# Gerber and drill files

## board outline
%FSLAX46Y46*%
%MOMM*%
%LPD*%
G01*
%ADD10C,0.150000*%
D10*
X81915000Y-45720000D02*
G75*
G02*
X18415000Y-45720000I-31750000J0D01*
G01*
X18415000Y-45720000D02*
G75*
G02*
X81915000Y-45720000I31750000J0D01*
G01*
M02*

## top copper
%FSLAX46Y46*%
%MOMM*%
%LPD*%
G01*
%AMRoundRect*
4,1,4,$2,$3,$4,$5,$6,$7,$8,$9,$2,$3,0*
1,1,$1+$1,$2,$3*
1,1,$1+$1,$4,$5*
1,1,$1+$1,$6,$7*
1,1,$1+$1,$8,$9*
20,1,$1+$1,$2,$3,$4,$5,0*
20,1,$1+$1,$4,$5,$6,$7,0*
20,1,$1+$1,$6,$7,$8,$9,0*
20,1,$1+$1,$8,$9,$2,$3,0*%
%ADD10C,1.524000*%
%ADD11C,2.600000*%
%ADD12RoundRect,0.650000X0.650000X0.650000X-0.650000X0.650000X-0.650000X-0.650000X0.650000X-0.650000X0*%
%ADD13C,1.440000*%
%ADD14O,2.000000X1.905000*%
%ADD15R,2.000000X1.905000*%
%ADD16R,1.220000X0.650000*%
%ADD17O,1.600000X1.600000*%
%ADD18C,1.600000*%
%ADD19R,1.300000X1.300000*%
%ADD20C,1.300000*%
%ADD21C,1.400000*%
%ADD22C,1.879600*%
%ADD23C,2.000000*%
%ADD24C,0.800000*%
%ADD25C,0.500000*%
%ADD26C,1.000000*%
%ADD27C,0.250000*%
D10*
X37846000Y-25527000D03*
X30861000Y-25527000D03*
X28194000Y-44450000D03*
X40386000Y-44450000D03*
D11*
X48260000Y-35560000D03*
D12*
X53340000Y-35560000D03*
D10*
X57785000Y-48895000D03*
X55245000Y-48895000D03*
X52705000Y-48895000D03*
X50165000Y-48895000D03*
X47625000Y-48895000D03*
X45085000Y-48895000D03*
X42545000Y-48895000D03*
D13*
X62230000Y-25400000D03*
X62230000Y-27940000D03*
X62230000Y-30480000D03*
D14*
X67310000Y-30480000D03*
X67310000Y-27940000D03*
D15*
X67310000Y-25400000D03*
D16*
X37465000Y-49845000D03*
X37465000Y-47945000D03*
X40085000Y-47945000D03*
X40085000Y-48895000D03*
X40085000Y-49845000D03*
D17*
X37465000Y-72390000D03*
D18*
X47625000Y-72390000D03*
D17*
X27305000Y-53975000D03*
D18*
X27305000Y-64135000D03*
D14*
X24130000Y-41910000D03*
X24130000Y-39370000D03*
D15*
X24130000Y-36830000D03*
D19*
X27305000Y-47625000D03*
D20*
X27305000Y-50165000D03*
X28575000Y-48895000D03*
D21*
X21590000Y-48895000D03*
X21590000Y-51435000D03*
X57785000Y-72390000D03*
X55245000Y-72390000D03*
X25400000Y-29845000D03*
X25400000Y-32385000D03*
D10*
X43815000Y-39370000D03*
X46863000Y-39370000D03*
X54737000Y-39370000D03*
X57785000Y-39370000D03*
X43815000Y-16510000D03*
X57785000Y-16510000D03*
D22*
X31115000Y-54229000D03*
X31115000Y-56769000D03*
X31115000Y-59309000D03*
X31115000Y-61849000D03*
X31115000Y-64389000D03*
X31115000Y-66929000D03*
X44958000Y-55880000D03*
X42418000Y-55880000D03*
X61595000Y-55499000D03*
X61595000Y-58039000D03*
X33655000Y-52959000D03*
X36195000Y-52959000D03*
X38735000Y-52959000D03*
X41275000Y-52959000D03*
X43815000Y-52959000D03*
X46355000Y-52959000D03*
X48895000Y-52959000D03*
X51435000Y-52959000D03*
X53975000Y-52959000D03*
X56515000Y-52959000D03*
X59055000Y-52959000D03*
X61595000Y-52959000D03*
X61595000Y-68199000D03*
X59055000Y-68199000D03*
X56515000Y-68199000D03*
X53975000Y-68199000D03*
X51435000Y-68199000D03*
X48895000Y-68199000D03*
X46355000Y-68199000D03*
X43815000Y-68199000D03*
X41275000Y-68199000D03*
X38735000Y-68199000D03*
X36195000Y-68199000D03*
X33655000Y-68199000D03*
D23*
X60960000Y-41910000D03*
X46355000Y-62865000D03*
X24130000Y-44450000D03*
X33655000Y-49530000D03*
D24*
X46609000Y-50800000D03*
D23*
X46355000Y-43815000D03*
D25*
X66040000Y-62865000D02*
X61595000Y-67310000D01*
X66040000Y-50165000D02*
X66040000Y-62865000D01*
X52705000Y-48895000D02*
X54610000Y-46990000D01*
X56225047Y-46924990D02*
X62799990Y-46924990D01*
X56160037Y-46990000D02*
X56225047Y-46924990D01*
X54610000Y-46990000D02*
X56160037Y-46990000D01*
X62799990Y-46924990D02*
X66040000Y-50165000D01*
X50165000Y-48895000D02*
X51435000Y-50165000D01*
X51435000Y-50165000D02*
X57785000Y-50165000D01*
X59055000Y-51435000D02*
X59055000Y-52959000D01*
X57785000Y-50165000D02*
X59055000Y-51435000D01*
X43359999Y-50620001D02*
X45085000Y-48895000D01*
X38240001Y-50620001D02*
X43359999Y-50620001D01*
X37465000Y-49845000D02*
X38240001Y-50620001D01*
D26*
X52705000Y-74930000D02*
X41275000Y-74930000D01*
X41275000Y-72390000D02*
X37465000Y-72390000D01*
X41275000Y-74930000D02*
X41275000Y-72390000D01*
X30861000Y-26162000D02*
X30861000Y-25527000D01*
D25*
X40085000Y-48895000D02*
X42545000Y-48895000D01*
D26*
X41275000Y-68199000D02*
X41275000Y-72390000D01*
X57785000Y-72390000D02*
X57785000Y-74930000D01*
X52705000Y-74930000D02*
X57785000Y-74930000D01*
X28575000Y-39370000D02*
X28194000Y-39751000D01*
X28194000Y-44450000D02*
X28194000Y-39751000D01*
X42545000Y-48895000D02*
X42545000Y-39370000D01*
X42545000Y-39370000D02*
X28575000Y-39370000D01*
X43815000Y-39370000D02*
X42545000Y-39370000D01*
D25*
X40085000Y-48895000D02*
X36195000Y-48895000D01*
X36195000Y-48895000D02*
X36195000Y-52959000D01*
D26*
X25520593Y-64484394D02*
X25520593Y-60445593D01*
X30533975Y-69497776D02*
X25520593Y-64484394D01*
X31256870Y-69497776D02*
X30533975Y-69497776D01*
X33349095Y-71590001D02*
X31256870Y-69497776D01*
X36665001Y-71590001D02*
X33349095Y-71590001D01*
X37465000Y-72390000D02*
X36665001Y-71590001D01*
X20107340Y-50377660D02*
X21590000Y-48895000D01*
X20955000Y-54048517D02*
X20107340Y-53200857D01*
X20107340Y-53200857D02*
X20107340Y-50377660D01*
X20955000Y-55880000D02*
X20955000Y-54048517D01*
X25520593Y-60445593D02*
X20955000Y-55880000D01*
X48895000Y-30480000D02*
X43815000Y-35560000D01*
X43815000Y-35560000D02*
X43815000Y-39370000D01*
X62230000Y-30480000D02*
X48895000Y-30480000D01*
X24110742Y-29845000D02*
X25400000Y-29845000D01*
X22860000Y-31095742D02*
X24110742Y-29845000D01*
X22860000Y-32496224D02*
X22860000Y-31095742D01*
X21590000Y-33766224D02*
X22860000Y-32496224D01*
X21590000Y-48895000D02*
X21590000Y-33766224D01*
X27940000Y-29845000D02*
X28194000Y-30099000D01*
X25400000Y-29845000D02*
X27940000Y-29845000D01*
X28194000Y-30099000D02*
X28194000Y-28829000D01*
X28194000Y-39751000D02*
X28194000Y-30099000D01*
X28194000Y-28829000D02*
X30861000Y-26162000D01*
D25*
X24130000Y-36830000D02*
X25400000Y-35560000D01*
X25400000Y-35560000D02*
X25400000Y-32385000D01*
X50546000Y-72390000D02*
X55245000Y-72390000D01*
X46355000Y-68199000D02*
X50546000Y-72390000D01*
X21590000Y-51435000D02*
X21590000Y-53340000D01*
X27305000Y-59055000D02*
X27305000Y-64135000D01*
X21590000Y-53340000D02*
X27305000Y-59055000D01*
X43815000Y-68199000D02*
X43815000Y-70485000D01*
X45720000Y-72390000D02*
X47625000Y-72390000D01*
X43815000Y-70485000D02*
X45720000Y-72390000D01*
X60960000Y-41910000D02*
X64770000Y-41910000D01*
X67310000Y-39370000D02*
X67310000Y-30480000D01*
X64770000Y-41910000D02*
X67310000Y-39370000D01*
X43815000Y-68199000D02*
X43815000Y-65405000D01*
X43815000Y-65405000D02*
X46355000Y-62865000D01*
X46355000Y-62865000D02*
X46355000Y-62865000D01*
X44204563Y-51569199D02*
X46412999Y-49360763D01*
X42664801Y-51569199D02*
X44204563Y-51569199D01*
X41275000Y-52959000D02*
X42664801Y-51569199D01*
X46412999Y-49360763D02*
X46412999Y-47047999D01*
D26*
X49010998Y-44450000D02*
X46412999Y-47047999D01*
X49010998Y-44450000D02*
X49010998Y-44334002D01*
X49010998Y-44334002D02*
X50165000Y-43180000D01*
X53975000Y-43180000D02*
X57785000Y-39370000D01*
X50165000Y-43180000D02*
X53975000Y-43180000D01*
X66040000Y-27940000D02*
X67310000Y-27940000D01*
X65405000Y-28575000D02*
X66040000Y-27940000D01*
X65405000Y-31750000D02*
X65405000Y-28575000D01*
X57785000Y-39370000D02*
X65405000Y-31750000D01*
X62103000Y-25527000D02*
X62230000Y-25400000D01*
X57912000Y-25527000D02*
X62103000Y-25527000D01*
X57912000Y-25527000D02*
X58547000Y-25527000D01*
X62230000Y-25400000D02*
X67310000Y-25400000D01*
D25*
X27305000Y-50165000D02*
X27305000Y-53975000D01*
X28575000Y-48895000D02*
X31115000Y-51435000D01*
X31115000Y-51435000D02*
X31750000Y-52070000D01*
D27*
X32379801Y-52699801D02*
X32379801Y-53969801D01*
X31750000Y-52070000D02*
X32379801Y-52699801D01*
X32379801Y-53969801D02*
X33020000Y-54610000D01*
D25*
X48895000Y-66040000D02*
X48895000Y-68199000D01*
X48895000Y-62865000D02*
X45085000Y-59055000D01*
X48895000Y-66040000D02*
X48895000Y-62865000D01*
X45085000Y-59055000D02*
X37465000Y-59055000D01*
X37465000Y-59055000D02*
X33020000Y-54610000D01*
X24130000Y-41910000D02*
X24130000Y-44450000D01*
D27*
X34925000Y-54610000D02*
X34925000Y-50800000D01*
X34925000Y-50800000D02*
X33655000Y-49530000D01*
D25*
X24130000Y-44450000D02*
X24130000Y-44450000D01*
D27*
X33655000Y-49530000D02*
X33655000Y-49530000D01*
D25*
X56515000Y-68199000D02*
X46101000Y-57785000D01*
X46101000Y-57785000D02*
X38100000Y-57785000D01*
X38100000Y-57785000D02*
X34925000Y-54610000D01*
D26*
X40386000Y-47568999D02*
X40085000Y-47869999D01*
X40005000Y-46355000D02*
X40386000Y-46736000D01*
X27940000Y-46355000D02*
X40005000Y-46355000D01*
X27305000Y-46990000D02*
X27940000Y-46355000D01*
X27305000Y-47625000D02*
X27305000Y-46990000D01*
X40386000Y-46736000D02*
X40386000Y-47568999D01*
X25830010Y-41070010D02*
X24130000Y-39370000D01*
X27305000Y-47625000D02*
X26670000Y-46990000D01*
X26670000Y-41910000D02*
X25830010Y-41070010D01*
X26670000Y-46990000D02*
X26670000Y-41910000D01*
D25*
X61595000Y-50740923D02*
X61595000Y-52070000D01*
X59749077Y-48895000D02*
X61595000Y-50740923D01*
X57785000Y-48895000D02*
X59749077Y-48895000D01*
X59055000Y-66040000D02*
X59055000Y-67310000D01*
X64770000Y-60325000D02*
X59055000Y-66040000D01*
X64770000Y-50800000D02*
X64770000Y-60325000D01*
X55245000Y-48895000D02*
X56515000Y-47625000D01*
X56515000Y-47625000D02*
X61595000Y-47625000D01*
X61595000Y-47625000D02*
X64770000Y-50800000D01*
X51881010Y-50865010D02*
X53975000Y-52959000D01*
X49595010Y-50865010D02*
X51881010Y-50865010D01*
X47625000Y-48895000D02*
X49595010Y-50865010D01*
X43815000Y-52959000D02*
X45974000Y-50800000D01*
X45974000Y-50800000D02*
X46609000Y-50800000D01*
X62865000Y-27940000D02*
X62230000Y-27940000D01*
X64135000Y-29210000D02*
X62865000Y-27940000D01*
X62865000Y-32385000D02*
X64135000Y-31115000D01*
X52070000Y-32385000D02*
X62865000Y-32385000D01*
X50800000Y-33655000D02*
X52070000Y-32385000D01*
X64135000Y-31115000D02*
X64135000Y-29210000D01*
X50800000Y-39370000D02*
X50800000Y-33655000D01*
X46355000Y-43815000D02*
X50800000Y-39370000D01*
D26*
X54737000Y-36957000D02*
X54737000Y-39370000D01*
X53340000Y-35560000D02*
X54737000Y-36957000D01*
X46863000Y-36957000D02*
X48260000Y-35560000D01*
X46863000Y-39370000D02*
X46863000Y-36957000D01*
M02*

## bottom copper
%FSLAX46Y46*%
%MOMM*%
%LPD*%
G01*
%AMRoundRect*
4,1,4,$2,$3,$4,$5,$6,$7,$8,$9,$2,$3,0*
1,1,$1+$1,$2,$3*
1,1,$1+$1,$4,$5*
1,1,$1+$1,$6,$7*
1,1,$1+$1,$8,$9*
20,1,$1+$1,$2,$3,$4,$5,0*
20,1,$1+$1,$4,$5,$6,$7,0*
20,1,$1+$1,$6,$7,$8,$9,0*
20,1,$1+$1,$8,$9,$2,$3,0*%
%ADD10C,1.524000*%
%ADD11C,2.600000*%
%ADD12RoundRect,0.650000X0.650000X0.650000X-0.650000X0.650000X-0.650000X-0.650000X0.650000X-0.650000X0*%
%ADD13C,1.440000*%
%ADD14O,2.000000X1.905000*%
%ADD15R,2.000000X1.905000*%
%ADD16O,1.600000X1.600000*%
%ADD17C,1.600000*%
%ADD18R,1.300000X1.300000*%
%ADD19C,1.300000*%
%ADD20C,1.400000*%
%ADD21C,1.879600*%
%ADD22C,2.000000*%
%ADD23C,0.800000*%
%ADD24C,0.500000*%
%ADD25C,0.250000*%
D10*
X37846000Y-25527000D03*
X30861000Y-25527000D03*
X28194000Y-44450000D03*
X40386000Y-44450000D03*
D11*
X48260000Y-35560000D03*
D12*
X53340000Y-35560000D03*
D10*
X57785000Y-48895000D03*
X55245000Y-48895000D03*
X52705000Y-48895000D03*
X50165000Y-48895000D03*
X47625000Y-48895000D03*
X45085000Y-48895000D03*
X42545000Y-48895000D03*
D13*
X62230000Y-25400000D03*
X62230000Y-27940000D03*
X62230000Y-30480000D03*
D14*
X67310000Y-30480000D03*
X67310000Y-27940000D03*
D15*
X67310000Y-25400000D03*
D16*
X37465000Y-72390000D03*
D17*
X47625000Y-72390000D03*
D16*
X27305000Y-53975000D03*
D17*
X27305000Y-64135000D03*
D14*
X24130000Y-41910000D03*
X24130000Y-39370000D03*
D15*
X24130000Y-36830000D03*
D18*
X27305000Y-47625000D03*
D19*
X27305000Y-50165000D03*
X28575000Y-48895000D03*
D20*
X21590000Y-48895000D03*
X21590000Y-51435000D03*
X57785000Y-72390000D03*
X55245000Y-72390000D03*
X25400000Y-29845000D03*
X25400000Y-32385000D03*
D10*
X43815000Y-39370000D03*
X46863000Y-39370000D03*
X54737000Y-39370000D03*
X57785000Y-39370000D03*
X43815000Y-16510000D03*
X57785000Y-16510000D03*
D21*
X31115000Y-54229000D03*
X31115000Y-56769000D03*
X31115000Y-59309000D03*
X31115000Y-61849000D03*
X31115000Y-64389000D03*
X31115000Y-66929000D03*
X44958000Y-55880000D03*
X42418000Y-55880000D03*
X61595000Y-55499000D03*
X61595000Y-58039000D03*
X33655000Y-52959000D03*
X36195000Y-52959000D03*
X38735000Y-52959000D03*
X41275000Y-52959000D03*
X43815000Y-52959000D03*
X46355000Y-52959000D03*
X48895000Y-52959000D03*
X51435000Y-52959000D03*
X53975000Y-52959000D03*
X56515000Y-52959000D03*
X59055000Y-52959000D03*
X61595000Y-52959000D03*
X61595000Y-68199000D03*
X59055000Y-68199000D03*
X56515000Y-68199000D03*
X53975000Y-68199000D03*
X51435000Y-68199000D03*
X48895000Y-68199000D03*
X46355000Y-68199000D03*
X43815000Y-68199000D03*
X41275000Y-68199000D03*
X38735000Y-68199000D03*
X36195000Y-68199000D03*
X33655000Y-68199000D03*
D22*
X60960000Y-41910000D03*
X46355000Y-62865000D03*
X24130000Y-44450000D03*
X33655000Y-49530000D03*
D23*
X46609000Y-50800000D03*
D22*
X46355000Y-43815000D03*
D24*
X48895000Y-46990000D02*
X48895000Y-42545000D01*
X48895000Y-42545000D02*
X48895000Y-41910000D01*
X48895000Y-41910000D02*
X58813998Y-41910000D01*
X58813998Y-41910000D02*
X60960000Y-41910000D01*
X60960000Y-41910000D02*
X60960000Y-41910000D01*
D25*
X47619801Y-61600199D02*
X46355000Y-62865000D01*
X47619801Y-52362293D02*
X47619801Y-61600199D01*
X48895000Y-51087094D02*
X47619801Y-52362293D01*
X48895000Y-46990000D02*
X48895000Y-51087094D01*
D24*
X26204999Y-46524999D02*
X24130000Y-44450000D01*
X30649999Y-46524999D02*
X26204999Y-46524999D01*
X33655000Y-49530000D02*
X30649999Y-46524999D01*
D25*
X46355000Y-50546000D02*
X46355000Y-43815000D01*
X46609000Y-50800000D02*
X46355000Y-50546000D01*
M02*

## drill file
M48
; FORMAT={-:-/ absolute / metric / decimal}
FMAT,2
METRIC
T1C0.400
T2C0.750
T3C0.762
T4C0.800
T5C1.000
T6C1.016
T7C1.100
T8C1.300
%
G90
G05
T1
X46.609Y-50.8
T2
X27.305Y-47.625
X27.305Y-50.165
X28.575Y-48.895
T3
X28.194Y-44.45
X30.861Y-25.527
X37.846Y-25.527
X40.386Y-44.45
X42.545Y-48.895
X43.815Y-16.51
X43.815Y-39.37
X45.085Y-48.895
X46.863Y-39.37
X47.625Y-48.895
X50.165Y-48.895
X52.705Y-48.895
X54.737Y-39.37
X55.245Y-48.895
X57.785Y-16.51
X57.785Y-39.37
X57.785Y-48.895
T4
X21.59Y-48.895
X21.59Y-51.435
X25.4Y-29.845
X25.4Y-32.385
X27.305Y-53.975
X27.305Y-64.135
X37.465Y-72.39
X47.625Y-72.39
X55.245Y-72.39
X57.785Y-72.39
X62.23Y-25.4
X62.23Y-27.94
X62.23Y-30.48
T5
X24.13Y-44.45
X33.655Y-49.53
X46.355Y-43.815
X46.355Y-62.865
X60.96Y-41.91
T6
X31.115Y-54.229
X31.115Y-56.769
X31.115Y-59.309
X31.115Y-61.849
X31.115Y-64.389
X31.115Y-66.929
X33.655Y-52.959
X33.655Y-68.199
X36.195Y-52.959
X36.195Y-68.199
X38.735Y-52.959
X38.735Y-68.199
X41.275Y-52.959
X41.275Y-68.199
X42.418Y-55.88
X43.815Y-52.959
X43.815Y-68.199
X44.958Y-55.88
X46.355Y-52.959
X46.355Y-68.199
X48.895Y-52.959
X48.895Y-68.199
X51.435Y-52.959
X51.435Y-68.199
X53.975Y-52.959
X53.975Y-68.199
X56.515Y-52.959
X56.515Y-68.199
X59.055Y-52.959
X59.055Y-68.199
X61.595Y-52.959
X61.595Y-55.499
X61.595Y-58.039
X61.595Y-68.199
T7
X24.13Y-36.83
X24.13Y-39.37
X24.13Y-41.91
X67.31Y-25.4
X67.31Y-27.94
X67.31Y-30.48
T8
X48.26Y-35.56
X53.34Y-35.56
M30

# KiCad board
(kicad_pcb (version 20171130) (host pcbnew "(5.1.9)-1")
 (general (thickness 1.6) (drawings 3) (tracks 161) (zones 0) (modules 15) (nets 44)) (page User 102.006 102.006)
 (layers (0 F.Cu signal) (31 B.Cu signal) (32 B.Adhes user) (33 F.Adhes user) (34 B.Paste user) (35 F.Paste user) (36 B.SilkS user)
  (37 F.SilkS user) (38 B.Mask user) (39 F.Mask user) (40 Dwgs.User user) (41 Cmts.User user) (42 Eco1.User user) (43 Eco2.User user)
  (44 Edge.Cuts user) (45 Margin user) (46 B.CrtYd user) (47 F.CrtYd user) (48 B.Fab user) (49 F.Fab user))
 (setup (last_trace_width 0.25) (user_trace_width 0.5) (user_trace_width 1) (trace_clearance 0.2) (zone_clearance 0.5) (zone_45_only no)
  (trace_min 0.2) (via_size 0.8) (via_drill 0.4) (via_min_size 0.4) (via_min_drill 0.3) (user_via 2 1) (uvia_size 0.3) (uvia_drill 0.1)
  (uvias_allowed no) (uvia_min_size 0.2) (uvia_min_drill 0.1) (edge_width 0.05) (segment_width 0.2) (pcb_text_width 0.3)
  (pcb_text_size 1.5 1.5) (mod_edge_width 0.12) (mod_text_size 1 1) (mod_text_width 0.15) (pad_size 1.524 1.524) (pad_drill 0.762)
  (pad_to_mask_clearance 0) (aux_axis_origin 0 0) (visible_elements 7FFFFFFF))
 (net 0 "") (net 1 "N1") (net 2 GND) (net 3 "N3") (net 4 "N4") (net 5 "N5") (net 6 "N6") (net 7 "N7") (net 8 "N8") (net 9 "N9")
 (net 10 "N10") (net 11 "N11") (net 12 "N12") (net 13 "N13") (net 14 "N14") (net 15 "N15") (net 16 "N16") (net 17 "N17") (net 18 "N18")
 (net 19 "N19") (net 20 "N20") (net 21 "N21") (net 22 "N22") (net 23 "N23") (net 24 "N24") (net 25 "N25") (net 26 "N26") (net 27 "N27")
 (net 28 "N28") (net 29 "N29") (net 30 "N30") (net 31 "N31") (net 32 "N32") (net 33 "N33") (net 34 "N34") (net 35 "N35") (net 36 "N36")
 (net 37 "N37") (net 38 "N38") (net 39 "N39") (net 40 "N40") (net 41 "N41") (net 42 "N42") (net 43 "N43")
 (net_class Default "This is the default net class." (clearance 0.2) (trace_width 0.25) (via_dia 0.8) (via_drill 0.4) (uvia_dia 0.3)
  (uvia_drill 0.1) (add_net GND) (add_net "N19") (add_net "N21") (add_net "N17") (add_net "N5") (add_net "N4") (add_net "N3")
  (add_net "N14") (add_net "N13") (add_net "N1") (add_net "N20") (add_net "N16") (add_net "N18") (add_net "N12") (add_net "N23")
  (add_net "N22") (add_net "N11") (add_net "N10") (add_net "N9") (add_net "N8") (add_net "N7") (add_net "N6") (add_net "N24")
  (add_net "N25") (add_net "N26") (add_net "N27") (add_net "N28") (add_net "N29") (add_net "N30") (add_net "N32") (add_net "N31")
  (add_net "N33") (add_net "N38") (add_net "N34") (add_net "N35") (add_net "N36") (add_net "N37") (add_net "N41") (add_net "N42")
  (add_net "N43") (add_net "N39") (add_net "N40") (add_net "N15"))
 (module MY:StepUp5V (layer F.Cu) (at 33.655 34.29 270)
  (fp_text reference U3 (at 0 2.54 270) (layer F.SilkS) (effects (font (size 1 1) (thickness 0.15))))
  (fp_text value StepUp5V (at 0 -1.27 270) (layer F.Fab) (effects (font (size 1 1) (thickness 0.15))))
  (pad 3 thru_hole circle (at -8.763 -4.191 270) (size 1.524 1.524) (drill 0.762) (layers *.Cu *.Mask) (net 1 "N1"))
  (pad 4 thru_hole circle (at -8.763 2.794 270) (size 1.524 1.524) (drill 0.762) (layers *.Cu *.Mask) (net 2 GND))
  (pad 2 thru_hole circle (at 10.16 5.461 270) (size 1.524 1.524) (drill 0.762) (layers *.Cu *.Mask) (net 2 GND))
  (pad 1 thru_hole circle (at 10.16 -6.731 270) (size 1.524 1.524) (drill 0.762) (layers *.Cu *.Mask) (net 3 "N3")))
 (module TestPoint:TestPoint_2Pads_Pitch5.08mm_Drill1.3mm (layer F.Cu) (at 53.34 35.56 180)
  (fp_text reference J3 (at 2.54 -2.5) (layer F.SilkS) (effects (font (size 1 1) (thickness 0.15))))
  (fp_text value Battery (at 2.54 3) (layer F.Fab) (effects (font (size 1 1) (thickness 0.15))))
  (pad 2 thru_hole circle (at 5.08 0 180) (size 2.6 2.6) (drill 1.3) (layers *.Cu *.Mask) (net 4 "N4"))
  (pad 1 thru_hole roundrect (at 0 0 180) (size 2.6 2.6) (drill 1.3) (layers *.Cu *.Mask) (roundrect_rratio 0.25) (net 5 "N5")))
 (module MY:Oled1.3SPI (layer F.Cu) (at 50.165 61.595)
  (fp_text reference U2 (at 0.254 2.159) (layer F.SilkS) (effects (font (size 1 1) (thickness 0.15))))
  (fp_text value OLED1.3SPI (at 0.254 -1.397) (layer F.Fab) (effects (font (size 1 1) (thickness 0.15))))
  (pad 7 thru_hole circle (at 7.62 -12.7) (size 1.524 1.524) (drill 0.762) (layers *.Cu *.Mask) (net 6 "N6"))
  (pad 6 thru_hole circle (at 5.08 -12.7) (size 1.524 1.524) (drill 0.762) (layers *.Cu *.Mask) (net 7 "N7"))
  (pad 5 thru_hole circle (at 2.54 -12.7) (size 1.524 1.524) (drill 0.762) (layers *.Cu *.Mask) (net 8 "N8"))
  (pad 4 thru_hole circle (at 0 -12.7) (size 1.524 1.524) (drill 0.762) (layers *.Cu *.Mask) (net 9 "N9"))
  (pad 3 thru_hole circle (at -2.54 -12.7) (size 1.524 1.524) (drill 0.762) (layers *.Cu *.Mask) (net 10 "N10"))
  (pad 2 thru_hole circle (at -5.08 -12.7) (size 1.524 1.524) (drill 0.762) (layers *.Cu *.Mask) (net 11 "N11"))
  (pad 1 thru_hole circle (at -7.62 -12.7) (size 1.524 1.524) (drill 0.762) (layers *.Cu *.Mask) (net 2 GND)))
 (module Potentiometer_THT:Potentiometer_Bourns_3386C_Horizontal (layer F.Cu) (at 62.23 25.4)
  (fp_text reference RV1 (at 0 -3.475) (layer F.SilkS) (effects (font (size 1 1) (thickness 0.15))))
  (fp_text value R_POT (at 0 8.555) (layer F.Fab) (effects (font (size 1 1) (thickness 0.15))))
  (pad 1 thru_hole circle (at 0 0) (size 1.44 1.44) (drill 0.8) (layers *.Cu *.Mask) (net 3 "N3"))
  (pad 2 thru_hole circle (at 0 2.54) (size 1.44 1.44) (drill 0.8) (layers *.Cu *.Mask) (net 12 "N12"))
  (pad 3 thru_hole circle (at 0 5.08) (size 1.44 1.44) (drill 0.8) (layers *.Cu *.Mask) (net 2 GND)))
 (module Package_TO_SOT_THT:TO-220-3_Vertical (layer F.Cu) (at 67.31 25.4 270)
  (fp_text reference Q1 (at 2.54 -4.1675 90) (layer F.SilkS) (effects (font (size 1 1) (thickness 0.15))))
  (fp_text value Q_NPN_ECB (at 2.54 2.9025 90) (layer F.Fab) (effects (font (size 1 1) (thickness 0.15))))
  (pad 3 thru_hole oval (at 5.08 0 270) (size 1.905 2) (drill 1.1) (layers *.Cu *.Mask) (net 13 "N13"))
  (pad 2 thru_hole oval (at 2.54 0 270) (size 1.905 2) (drill 1.1) (layers *.Cu *.Mask) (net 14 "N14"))
  (pad 1 thru_hole rect (at 0 0 270) (size 1.905 2) (drill 1.1) (layers *.Cu *.Mask) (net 3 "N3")))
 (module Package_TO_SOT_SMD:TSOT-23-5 (layer F.Cu) (at 38.775 48.895 180)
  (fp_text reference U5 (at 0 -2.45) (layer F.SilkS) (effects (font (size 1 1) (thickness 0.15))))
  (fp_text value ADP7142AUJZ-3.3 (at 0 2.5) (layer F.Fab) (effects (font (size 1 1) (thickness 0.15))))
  (pad 5 smd rect (at 1.31 -0.95 180) (size 1.22 0.65) (layers F.Cu F.Paste F.Mask) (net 11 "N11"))
  (pad 4 smd rect (at 1.31 0.95 180) (size 1.22 0.65) (layers F.Cu F.Paste F.Mask) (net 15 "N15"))
  (pad 3 smd rect (at -1.31 0.95 180) (size 1.22 0.65) (layers F.Cu F.Paste F.Mask) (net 1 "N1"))
  (pad 2 smd rect (at -1.31 0 180) (size 1.22 0.65) (layers F.Cu F.Paste F.Mask) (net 2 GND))
  (pad 1 smd rect (at -1.31 -0.95 180) (size 1.22 0.65) (layers F.Cu F.Paste F.Mask) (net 1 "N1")))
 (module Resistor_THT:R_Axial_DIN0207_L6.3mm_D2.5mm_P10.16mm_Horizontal (layer F.Cu) (at 47.625 72.39 180)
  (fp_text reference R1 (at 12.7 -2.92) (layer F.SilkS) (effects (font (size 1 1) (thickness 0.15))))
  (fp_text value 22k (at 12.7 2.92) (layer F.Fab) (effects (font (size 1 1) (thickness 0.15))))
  (pad 2 thru_hole oval (at 10.16 0 180) (size 1.6 1.6) (drill 0.8) (layers *.Cu *.Mask) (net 2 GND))
  (pad 1 thru_hole circle (at 0 0 180) (size 1.6 1.6) (drill 0.8) (layers *.Cu *.Mask) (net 13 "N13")))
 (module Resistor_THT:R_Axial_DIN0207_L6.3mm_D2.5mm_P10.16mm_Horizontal (layer F.Cu) (at 27.305 64.135 90)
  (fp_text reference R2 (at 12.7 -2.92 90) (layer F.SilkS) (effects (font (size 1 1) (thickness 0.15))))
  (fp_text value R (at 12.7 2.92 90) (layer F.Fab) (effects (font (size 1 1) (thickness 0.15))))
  (pad 2 thru_hole oval (at 10.16 0 90) (size 1.6 1.6) (drill 0.8) (layers *.Cu *.Mask) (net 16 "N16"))
  (pad 1 thru_hole circle (at 0 0 90) (size 1.6 1.6) (drill 0.8) (layers *.Cu *.Mask) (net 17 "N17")))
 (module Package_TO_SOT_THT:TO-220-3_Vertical (layer F.Cu) (at 24.13 36.83 270)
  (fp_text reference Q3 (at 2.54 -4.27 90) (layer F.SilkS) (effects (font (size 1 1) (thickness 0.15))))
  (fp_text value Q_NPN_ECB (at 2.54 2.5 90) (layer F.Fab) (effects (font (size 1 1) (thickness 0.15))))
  (pad 3 thru_hole oval (at 5.08 0 270) (size 1.905 2) (drill 1.1) (layers *.Cu *.Mask) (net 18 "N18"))
  (pad 2 thru_hole oval (at 2.54 0 270) (size 1.905 2) (drill 1.1) (layers *.Cu *.Mask) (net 1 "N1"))
  (pad 1 thru_hole rect (at 0 0 270) (size 1.905 2) (drill 1.1) (layers *.Cu *.Mask) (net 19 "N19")))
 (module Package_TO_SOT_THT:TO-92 (layer F.Cu) (at 27.305 47.625 270)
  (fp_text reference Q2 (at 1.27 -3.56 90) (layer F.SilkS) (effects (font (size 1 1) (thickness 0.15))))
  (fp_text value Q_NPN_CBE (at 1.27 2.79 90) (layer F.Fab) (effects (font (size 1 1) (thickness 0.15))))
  (pad 1 thru_hole rect (at 0 0 270) (size 1.3 1.3) (drill 0.75) (layers *.Cu *.Mask) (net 1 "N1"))
  (pad 3 thru_hole circle (at 2.54 0 270) (size 1.3 1.3) (drill 0.75) (layers *.Cu *.Mask) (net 16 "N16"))
  (pad 2 thru_hole circle (at 1.27 -1.27 270) (size 1.3 1.3) (drill 0.75) (layers *.Cu *.Mask) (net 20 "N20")))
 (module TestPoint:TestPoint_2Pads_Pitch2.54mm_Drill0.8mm (layer F.Cu) (at 21.59 51.435 90)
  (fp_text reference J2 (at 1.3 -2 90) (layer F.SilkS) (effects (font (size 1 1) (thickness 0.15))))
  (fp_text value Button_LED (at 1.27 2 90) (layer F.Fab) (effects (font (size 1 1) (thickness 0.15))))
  (pad 2 thru_hole circle (at 2.54 0 90) (size 1.4 1.4) (drill 0.8) (layers *.Cu *.Mask) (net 2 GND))
  (pad 1 thru_hole circle (at 0 0 90) (size 1.4 1.4) (drill 0.8) (layers *.Cu *.Mask) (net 17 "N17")))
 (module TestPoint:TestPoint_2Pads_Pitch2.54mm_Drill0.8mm (layer F.Cu) (at 55.245 72.39)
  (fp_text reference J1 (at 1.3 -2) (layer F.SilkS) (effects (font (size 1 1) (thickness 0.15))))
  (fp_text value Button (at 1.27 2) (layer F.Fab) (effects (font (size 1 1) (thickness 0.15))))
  (pad 2 thru_hole circle (at 2.54 0) (size 1.4 1.4) (drill 0.8) (layers *.Cu *.Mask) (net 2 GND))
  (pad 1 thru_hole circle (at 0 0) (size 1.4 1.4) (drill 0.8) (layers *.Cu *.Mask) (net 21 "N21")))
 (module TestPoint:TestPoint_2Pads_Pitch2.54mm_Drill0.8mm (layer F.Cu) (at 25.4 32.385 90)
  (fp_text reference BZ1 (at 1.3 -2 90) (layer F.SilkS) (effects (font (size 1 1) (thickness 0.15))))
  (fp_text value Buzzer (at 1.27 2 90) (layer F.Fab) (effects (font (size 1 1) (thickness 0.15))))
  (pad 2 thru_hole circle (at 2.54 0 90) (size 1.4 1.4) (drill 0.8) (layers *.Cu *.Mask) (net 2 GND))
  (pad 1 thru_hole circle (at 0 0 90) (size 1.4 1.4) (drill 0.8) (layers *.Cu *.Mask) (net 19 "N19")))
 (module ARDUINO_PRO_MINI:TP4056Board (layer F.Cu) (at 46.355 27.94 270)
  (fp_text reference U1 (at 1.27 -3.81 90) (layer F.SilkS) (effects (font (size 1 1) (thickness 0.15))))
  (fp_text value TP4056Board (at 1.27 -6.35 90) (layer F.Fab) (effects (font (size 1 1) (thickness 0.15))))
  (pad 6 thru_hole circle (at 11.43 2.54 270) (size 1.524 1.524) (drill 0.762) (layers *.Cu *.Mask) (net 2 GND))
  (pad 5 thru_hole circle (at 11.43 -0.508 270) (size 1.524 1.524) (drill 0.762) (layers *.Cu *.Mask) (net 4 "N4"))
  (pad 4 thru_hole circle (at 11.43 -8.382 270) (size 1.524 1.524) (drill 0.762) (layers *.Cu *.Mask) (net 5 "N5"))
  (pad 3 thru_hole circle (at 11.43 -11.43 270) (size 1.524 1.524) (drill 0.762) (layers *.Cu *.Mask) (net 14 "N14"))
  (pad 2 thru_hole circle (at -11.43 2.54 270) (size 1.524 1.524) (drill 0.762) (layers *.Cu *.Mask) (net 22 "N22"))
  (pad 1 thru_hole circle (at -11.43 -11.43 270) (size 1.524 1.524) (drill 0.762) (layers *.Cu *.Mask) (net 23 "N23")))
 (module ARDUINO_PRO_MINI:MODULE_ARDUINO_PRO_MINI (layer F.Cu) (at 46.355 60.579 90)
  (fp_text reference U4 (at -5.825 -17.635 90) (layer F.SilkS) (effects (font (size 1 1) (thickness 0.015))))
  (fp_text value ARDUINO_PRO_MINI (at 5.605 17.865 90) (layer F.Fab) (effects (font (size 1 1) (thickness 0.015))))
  (pad JP1_1 thru_hole circle (at 6.35 -15.24 90) (size 1.8796 1.8796) (drill 1.016) (layers *.Cu *.Mask) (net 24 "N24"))
  (pad JP1_2 thru_hole circle (at 3.81 -15.24 90) (size 1.8796 1.8796) (drill 1.016) (layers *.Cu *.Mask) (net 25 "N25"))
  (pad JP1_3 thru_hole circle (at 1.27 -15.24 90) (size 1.8796 1.8796) (drill 1.016) (layers *.Cu *.Mask) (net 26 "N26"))
  (pad JP1_4 thru_hole circle (at -1.27 -15.24 90) (size 1.8796 1.8796) (drill 1.016) (layers *.Cu *.Mask) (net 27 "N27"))
  (pad JP1_5 thru_hole circle (at -3.81 -15.24 90) (size 1.8796 1.8796) (drill 1.016) (layers *.Cu *.Mask) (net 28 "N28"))
  (pad JP1_6 thru_hole circle (at -6.35 -15.24 90) (size 1.8796 1.8796) (drill 1.016) (layers *.Cu *.Mask) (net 28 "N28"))
  (pad JP2_1 thru_hole circle (at 4.699 -1.397 90) (size 1.8796 1.8796) (drill 1.016) (layers *.Cu *.Mask) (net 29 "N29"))
  (pad JP2_2 thru_hole circle (at 4.699 -3.937 90) (size 1.8796 1.8796) (drill 1.016) (layers *.Cu *.Mask) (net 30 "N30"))
  (pad JP3_2 thru_hole circle (at 5.08 15.24 90) (size 1.8796 1.8796) (drill 1.016) (layers *.Cu *.Mask) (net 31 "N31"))
  (pad JP3_1 thru_hole circle (at 2.54 15.24 90) (size 1.8796 1.8796) (drill 1.016) (layers *.Cu *.Mask) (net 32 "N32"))
  (pad JP6_1 thru_hole circle (at 7.62 -12.7 90) (size 1.8796 1.8796) (drill 1.016) (layers *.Cu *.Mask) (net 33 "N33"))
  (pad JP6_2 thru_hole circle (at 7.62 -10.16 90) (size 1.8796 1.8796) (drill 1.016) (layers *.Cu *.Mask) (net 2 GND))
  (pad JP6_3 thru_hole circle (at 7.62 -7.62 90) (size 1.8796 1.8796) (drill 1.016) (layers *.Cu *.Mask) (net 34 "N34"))
  (pad JP6_4 thru_hole circle (at 7.62 -5.08 90) (size 1.8796 1.8796) (drill 1.016) (layers *.Cu *.Mask) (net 14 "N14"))
  (pad JP6_5 thru_hole circle (at 7.62 -2.54 90) (size 1.8796 1.8796) (drill 1.016) (layers *.Cu *.Mask) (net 12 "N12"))
  (pad JP6_6 thru_hole circle (at 7.62 0 90) (size 1.8796 1.8796) (drill 1.016) (layers *.Cu *.Mask) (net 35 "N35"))
  (pad JP6_7 thru_hole circle (at 7.62 2.54 90) (size 1.8796 1.8796) (drill 1.016) (layers *.Cu *.Mask) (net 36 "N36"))
  (pad JP6_8 thru_hole circle (at 7.62 5.08 90) (size 1.8796 1.8796) (drill 1.016) (layers *.Cu *.Mask) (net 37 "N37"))
  (pad JP6_9 thru_hole circle (at 7.62 7.62 90) (size 1.8796 1.8796) (drill 1.016) (layers *.Cu *.Mask) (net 10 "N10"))
  (pad JP6_10 thru_hole circle (at 7.62 10.16 90) (size 1.8796 1.8796) (drill 1.016) (layers *.Cu *.Mask) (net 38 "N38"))
  (pad JP6_11 thru_hole circle (at 7.62 12.7 90) (size 1.8796 1.8796) (drill 1.016) (layers *.Cu *.Mask) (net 9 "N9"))
  (pad JP6_12 thru_hole circle (at 7.62 15.24 90) (size 1.8796 1.8796) (drill 1.016) (layers *.Cu *.Mask) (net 6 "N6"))
  (pad JP7_1 thru_hole circle (at -7.62 15.24 90) (size 1.8796 1.8796) (drill 1.016) (layers *.Cu *.Mask) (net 8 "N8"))
  (pad JP7_2 thru_hole circle (at -7.62 12.7 90) (size 1.8796 1.8796) (drill 1.016) (layers *.Cu *.Mask) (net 7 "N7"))
  (pad JP7_3 thru_hole circle (at -7.62 10.16 90) (size 1.8796 1.8796) (drill 1.016) (layers *.Cu *.Mask) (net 18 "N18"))
  (pad JP7_4 thru_hole circle (at -7.62 7.62 90) (size 1.8796 1.8796) (drill 1.016) (layers *.Cu *.Mask) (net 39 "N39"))
  (pad JP7_5 thru_hole circle (at -7.62 5.08 90) (size 1.8796 1.8796) (drill 1.016) (layers *.Cu *.Mask) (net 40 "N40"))
  (pad JP7_6 thru_hole circle (at -7.62 2.54 90) (size 1.8796 1.8796) (drill 1.016) (layers *.Cu *.Mask) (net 20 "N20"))
  (pad JP7_7 thru_hole circle (at -7.62 0 90) (size 1.8796 1.8796) (drill 1.016) (layers *.Cu *.Mask) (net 21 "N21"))
  (pad JP7_8 thru_hole circle (at -7.62 -2.54 90) (size 1.8796 1.8796) (drill 1.016) (layers *.Cu *.Mask) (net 13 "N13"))
  (pad JP7_9 thru_hole circle (at -7.62 -5.08 90) (size 1.8796 1.8796) (drill 1.016) (layers *.Cu *.Mask) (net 2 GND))
  (pad JP7_10 thru_hole circle (at -7.62 -7.62 90) (size 1.8796 1.8796) (drill 1.016) (layers *.Cu *.Mask) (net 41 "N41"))
  (pad JP7_11 thru_hole circle (at -7.62 -10.16 90) (size 1.8796 1.8796) (drill 1.016) (layers *.Cu *.Mask) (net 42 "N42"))
  (pad JP7_12 thru_hole circle (at -7.62 -12.7 90) (size 1.8796 1.8796) (drill 1.016) (layers *.Cu *.Mask) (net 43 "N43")))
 (gr_circle (center 50.165 45.72) (end 81.915 45.72) (layer Edge.Cuts) (width 0.15))
 (segment (start 66.04 62.865) (end 61.595 67.31) (width 0.5) (layer F.Cu) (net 8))
 (segment (start 66.04 50.165) (end 66.04 62.865) (width 0.5) (layer F.Cu) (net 8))
 (segment (start 52.705 48.895) (end 54.61 46.99) (width 0.5) (layer F.Cu) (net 8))
 (segment (start 56.225047 46.92499) (end 62.79999 46.92499) (width 0.5) (layer F.Cu) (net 8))
 (segment (start 56.160037 46.99) (end 56.225047 46.92499) (width 0.5) (layer F.Cu) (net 8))
 (segment (start 54.61 46.99) (end 56.160037 46.99) (width 0.5) (layer F.Cu) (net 8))
 (segment (start 62.79999 46.92499) (end 66.04 50.165) (width 0.5) (layer F.Cu) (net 8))
 (segment (start 50.165 48.895) (end 51.435 50.165) (width 0.5) (layer F.Cu) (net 9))
 (segment (start 51.435 50.165) (end 57.785 50.165) (width 0.5) (layer F.Cu) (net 9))
 (segment (start 59.055 51.435) (end 59.055 52.959) (width 0.5) (layer F.Cu) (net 9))
 (segment (start 57.785 50.165) (end 59.055 51.435) (width 0.5) (layer F.Cu) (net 9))
 (segment (start 43.359999 50.620001) (end 45.085 48.895) (width 0.5) (layer F.Cu) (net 11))
 (segment (start 38.240001 50.620001) (end 43.359999 50.620001) (width 0.5) (layer F.Cu) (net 11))
 (segment (start 37.465 49.845) (end 38.240001 50.620001) (width 0.5) (layer F.Cu) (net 11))
 (segment (start 52.705 74.93) (end 41.275 74.93) (width 1) (layer F.Cu) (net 2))
 (segment (start 41.275 72.39) (end 37.465 72.39) (width 1) (layer F.Cu) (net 2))
 (segment (start 41.275 74.93) (end 41.275 72.39) (width 1) (layer F.Cu) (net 2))
 (segment (start 30.861 26.162) (end 30.861 25.527) (width 1) (layer F.Cu) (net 2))
 (segment (start 40.085 48.895) (end 42.545 48.895) (width 0.5) (layer F.Cu) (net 2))
 (segment (start 41.275 68.199) (end 41.275 72.39) (width 1) (layer F.Cu) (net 2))
 (segment (start 57.785 72.39) (end 57.785 74.93) (width 1) (layer F.Cu) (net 2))
 (segment (start 52.705 74.93) (end 57.785 74.93) (width 1) (layer F.Cu) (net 2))
 (segment (start 28.575 39.37) (end 28.194 39.751) (width 1) (layer F.Cu) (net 2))
 (segment (start 28.194 44.45) (end 28.194 39.751) (width 1) (layer F.Cu) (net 2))
 (segment (start 42.545 48.895) (end 42.545 39.37) (width 1) (layer F.Cu) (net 2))
 (segment (start 42.545 39.37) (end 28.575 39.37) (width 1) (layer F.Cu) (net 2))
 (segment (start 43.815 39.37) (end 42.545 39.37) (width 1) (layer F.Cu) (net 2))
 (segment (start 40.085 48.895) (end 36.195 48.895) (width 0.5) (layer F.Cu) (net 2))
 (segment (start 36.195 48.895) (end 36.195 52.959) (width 0.5) (layer F.Cu) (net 2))
 (segment (start 25.520593 64.484394) (end 25.520593 60.445593) (width 1) (layer F.Cu) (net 2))
 (segment (start 30.533975 69.497776) (end 25.520593 64.484394) (width 1) (layer F.Cu) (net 2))
 (segment (start 31.25687 69.497776) (end 30.533975 69.497776) (width 1) (layer F.Cu) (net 2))
 (segment (start 33.349095 71.590001) (end 31.25687 69.497776) (width 1) (layer F.Cu) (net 2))
 (segment (start 36.665001 71.590001) (end 33.349095 71.590001) (width 1) (layer F.Cu) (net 2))
 (segment (start 37.465 72.39) (end 36.665001 71.590001) (width 1) (layer F.Cu) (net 2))
 (segment (start 20.10734 50.37766) (end 21.59 48.895) (width 1) (layer F.Cu) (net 2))
 (segment (start 20.955 54.048517) (end 20.10734 53.200857) (width 1) (layer F.Cu) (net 2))
 (segment (start 20.10734 53.200857) (end 20.10734 50.37766) (width 1) (layer F.Cu) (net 2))
 (segment (start 20.955 55.88) (end 20.955 54.048517) (width 1) (layer F.Cu) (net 2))
 (segment (start 25.520593 60.445593) (end 20.955 55.88) (width 1) (layer F.Cu) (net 2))
 (segment (start 48.895 30.48) (end 43.815 35.56) (width 1) (layer F.Cu) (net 2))
 (segment (start 43.815 35.56) (end 43.815 39.37) (width 1) (layer F.Cu) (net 2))
 (segment (start 62.23 30.48) (end 48.895 30.48) (width 1) (layer F.Cu) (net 2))
 (segment (start 24.110742 29.845) (end 25.4 29.845) (width 1) (layer F.Cu) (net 2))
 (segment (start 22.86 31.095742) (end 24.110742 29.845) (width 1) (layer F.Cu) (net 2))
 (segment (start 22.86 32.496224) (end 22.86 31.095742) (width 1) (layer F.Cu) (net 2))
 (segment (start 21.59 33.766224) (end 22.86 32.496224) (width 1) (layer F.Cu) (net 2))
 (segment (start 21.59 48.895) (end 21.59 33.766224) (width 1) (layer F.Cu) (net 2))
 (segment (start 27.94 29.845) (end 28.194 30.099) (width 1) (layer F.Cu) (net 2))
 (segment (start 25.4 29.845) (end 27.94 29.845) (width 1) (layer F.Cu) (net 2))
 (segment (start 28.194 30.099) (end 28.194 28.829) (width 1) (layer F.Cu) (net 2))
 (segment (start 28.194 39.751) (end 28.194 30.099) (width 1) (layer F.Cu) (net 2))
 (segment (start 28.194 28.829) (end 30.861 26.162) (width 1) (layer F.Cu) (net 2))
 (segment (start 24.13 36.83) (end 25.4 35.56) (width 0.5) (layer F.Cu) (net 19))
 (segment (start 25.4 35.56) (end 25.4 32.385) (width 0.5) (layer F.Cu) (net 19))
 (segment (start 50.546 72.39) (end 55.245 72.39) (width 0.5) (layer F.Cu) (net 21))
 (segment (start 46.355 68.199) (end 50.546 72.39) (width 0.5) (layer F.Cu) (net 21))
 (segment (start 21.59 51.435) (end 21.59 53.34) (width 0.5) (layer F.Cu) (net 17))
 (segment (start 27.305 59.055) (end 27.305 64.135) (width 0.5) (layer F.Cu) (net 17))
 (segment (start 21.59 53.34) (end 27.305 59.055) (width 0.5) (layer F.Cu) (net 17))
 (segment (start 43.815 68.199) (end 43.815 70.485) (width 0.5) (layer F.Cu) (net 13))
 (segment (start 45.72 72.39) (end 47.625 72.39) (width 0.5) (layer F.Cu) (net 13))
 (segment (start 43.815 70.485) (end 45.72 72.39) (width 0.5) (layer F.Cu) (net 13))
 (segment (start 48.895 46.99) (end 48.895 42.545) (width 0.5) (layer B.Cu) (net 13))
 (segment (start 48.895 42.545) (end 48.895 41.91) (width 0.5) (layer B.Cu) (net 13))
 (segment (start 48.895 41.91) (end 58.813998 41.91) (width 0.5) (layer B.Cu) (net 13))
 (segment (start 58.813998 41.91) (end 60.96 41.91) (width 0.5) (layer B.Cu) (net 13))
 (segment (start 60.96 41.91) (end 60.96 41.91) (width 0.5) (layer B.Cu) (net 13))
 (via (at 60.96 41.91) (size 2) (drill 1) (layers F.Cu B.Cu) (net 13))
 (segment (start 60.96 41.91) (end 64.77 41.91) (width 0.5) (layer F.Cu) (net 13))
 (segment (start 67.31 39.37) (end 67.31 30.48) (width 0.5) (layer F.Cu) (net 13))
 (segment (start 64.77 41.91) (end 67.31 39.37) (width 0.5) (layer F.Cu) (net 13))
 (segment (start 43.815 68.199) (end 43.815 65.405) (width 0.5) (layer F.Cu) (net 13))
 (segment (start 43.815 65.405) (end 46.355 62.865) (width 0.5) (layer F.Cu) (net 13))
 (segment (start 46.355 62.865) (end 46.355 62.865) (width 0.5) (layer F.Cu) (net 13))
 (via (at 46.355 62.865) (size 2) (drill 1) (layers F.Cu B.Cu) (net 13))
 (segment (start 47.619801 61.600199) (end 46.355 62.865) (width 0.25) (layer B.Cu) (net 13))
 (segment (start 47.619801 52.362293) (end 47.619801 61.600199) (width 0.25) (layer B.Cu) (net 13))
 (segment (start 48.895 51.087094) (end 47.619801 52.362293) (width 0.25) (layer B.Cu) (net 13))
 (segment (start 48.895 46.99) (end 48.895 51.087094) (width 0.25) (layer B.Cu) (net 13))
 (segment (start 44.204563 51.569199) (end 46.412999 49.360763) (width 0.5) (layer F.Cu) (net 14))
 (segment (start 42.664801 51.569199) (end 44.204563 51.569199) (width 0.5) (layer F.Cu) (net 14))
 (segment (start 41.275 52.959) (end 42.664801 51.569199) (width 0.5) (layer F.Cu) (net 14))
 (segment (start 46.412999 49.360763) (end 46.412999 47.047999) (width 0.5) (layer F.Cu) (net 14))
 (segment (start 49.010998 44.45) (end 46.412999 47.047999) (width 1) (layer F.Cu) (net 14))
 (segment (start 49.010998 44.45) (end 49.010998 44.334002) (width 1) (layer F.Cu) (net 14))
 (segment (start 49.010998 44.334002) (end 50.165 43.18) (width 1) (layer F.Cu) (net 14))
 (segment (start 53.975 43.18) (end 57.785 39.37) (width 1) (layer F.Cu) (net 14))
 (segment (start 50.165 43.18) (end 53.975 43.18) (width 1) (layer F.Cu) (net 14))
 (segment (start 66.04 27.94) (end 67.31 27.94) (width 1) (layer F.Cu) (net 14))
 (segment (start 65.405 28.575) (end 66.04 27.94) (width 1) (layer F.Cu) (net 14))
 (segment (start 65.405 31.75) (end 65.405 28.575) (width 1) (layer F.Cu) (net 14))
 (segment (start 57.785 39.37) (end 65.405 31.75) (width 1) (layer F.Cu) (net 14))
 (segment (start 62.103 25.527) (end 62.23 25.4) (width 1) (layer F.Cu) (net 3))
 (segment (start 57.912 25.527) (end 62.103 25.527) (width 1) (layer F.Cu) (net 3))
 (segment (start 57.912 25.527) (end 58.547 25.527) (width 1) (layer F.Cu) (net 3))
 (segment (start 62.23 25.4) (end 67.31 25.4) (width 1) (layer F.Cu) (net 3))
 (segment (start 27.305 50.165) (end 27.305 53.975) (width 0.5) (layer F.Cu) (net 16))
 (segment (start 28.575 48.895) (end 31.115 51.435) (width 0.5) (layer F.Cu) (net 20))
 (segment (start 31.115 51.435) (end 31.75 52.07) (width 0.5) (layer F.Cu) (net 20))
 (segment (start 32.379801 52.699801) (end 32.379801 53.969801) (width 0.25) (layer F.Cu) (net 20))
 (segment (start 31.75 52.07) (end 32.379801 52.699801) (width 0.25) (layer F.Cu) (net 20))
 (segment (start 32.379801 53.969801) (end 33.02 54.61) (width 0.25) (layer F.Cu) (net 20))
 (segment (start 48.895 66.04) (end 48.895 68.199) (width 0.5) (layer F.Cu) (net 20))
 (segment (start 48.895 62.865) (end 45.085 59.055) (width 0.5) (layer F.Cu) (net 20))
 (segment (start 48.895 66.04) (end 48.895 62.865) (width 0.5) (layer F.Cu) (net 20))
 (segment (start 45.085 59.055) (end 37.465 59.055) (width 0.5) (layer F.Cu) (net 20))
 (segment (start 37.465 59.055) (end 33.02 54.61) (width 0.5) (layer F.Cu) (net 20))
 (segment (start 24.13 41.91) (end 24.13 44.45) (width 0.5) (layer F.Cu) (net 18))
 (segment (start 34.925 54.61) (end 34.925 50.8) (width 0.25) (layer F.Cu) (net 18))
 (segment (start 34.925 50.8) (end 33.655 49.53) (width 0.25) (layer F.Cu) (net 18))
 (segment (start 24.13 44.45) (end 24.13 44.45) (width 0.5) (layer F.Cu) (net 18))
 (via (at 24.13 44.45) (size 2) (drill 1) (layers F.Cu B.Cu) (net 18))
 (segment (start 33.655 49.53) (end 33.655 49.53) (width 0.25) (layer F.Cu) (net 18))
 (via (at 33.655 49.53) (size 2) (drill 1) (layers F.Cu B.Cu) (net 18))
 (segment (start 26.204999 46.524999) (end 24.13 44.45) (width 0.5) (layer B.Cu) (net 18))
 (segment (start 30.649999 46.524999) (end 26.204999 46.524999) (width 0.5) (layer B.Cu) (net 18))
 (segment (start 33.655 49.53) (end 30.649999 46.524999) (width 0.5) (layer B.Cu) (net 18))
 (segment (start 56.515 68.199) (end 46.101 57.785) (width 0.5) (layer F.Cu) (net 18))
 (segment (start 46.101 57.785) (end 38.1 57.785) (width 0.5) (layer F.Cu) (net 18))
 (segment (start 38.1 57.785) (end 34.925 54.61) (width 0.5) (layer F.Cu) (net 18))
 (segment (start 40.386 47.568999) (end 40.085 47.869999) (width 1) (layer F.Cu) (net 1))
 (segment (start 40.005 46.355) (end 40.386 46.736) (width 1) (layer F.Cu) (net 1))
 (segment (start 27.94 46.355) (end 40.005 46.355) (width 1) (layer F.Cu) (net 1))
 (segment (start 27.305 46.99) (end 27.94 46.355) (width 1) (layer F.Cu) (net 1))
 (segment (start 27.305 47.625) (end 27.305 46.99) (width 1) (layer F.Cu) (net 1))
 (segment (start 40.386 46.736) (end 40.386 47.568999) (width 1) (layer F.Cu) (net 1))
 (segment (start 25.83001 41.07001) (end 24.13 39.37) (width 1) (layer F.Cu) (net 1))
 (segment (start 27.305 47.625) (end 26.67 46.99) (width 1) (layer F.Cu) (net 1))
 (segment (start 26.67 41.91) (end 25.83001 41.07001) (width 1) (layer F.Cu) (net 1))
 (segment (start 26.67 46.99) (end 26.67 41.91) (width 1) (layer F.Cu) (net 1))
 (segment (start 61.595 50.740923) (end 61.595 52.07) (width 0.5) (layer F.Cu) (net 6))
 (segment (start 59.749077 48.895) (end 61.595 50.740923) (width 0.5) (layer F.Cu) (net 6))
 (segment (start 57.785 48.895) (end 59.749077 48.895) (width 0.5) (layer F.Cu) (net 6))
 (segment (start 59.055 66.04) (end 59.055 67.31) (width 0.5) (layer F.Cu) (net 7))
 (segment (start 64.77 60.325) (end 59.055 66.04) (width 0.5) (layer F.Cu) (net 7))
 (segment (start 64.77 50.8) (end 64.77 60.325) (width 0.5) (layer F.Cu) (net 7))
 (segment (start 55.245 48.895) (end 56.515 47.625) (width 0.5) (layer F.Cu) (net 7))
 (segment (start 56.515 47.625) (end 61.595 47.625) (width 0.5) (layer F.Cu) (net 7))
 (segment (start 61.595 47.625) (end 64.77 50.8) (width 0.5) (layer F.Cu) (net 7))
 (segment (start 51.88101 50.86501) (end 53.975 52.959) (width 0.5) (layer F.Cu) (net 10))
 (segment (start 49.59501 50.86501) (end 51.88101 50.86501) (width 0.5) (layer F.Cu) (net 10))
 (segment (start 47.625 48.895) (end 49.59501 50.86501) (width 0.5) (layer F.Cu) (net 10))
 (segment (start 43.815 52.959) (end 45.974 50.8) (width 0.5) (layer F.Cu) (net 12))
 (via (at 46.609 50.8) (size 0.8) (drill 0.4) (layers F.Cu B.Cu) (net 12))
 (segment (start 45.974 50.8) (end 46.609 50.8) (width 0.5) (layer F.Cu) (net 12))
 (via (at 46.355 43.815) (size 2) (drill 1) (layers F.Cu B.Cu) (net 12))
 (segment (start 46.355 50.546) (end 46.355 43.815) (width 0.25) (layer B.Cu) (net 12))
 (segment (start 46.609 50.8) (end 46.355 50.546) (width 0.25) (layer B.Cu) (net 12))
 (segment (start 62.865 27.94) (end 62.23 27.94) (width 0.5) (layer F.Cu) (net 12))
 (segment (start 64.135 29.21) (end 62.865 27.94) (width 0.5) (layer F.Cu) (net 12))
 (segment (start 62.865 32.385) (end 64.135 31.115) (width 0.5) (layer F.Cu) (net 12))
 (segment (start 52.07 32.385) (end 62.865 32.385) (width 0.5) (layer F.Cu) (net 12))
 (segment (start 50.8 33.655) (end 52.07 32.385) (width 0.5) (layer F.Cu) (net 12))
 (segment (start 64.135 31.115) (end 64.135 29.21) (width 0.5) (layer F.Cu) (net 12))
 (segment (start 50.8 39.37) (end 50.8 33.655) (width 0.5) (layer F.Cu) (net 12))
 (segment (start 46.355 43.815) (end 50.8 39.37) (width 0.5) (layer F.Cu) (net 12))
 (segment (start 54.737 36.957) (end 54.737 39.37) (width 1) (layer F.Cu) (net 5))
 (segment (start 53.34 35.56) (end 54.737 36.957) (width 1) (layer F.Cu) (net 5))
 (segment (start 46.863 36.957) (end 48.26 35.56) (width 1) (layer F.Cu) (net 4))
 (segment (start 46.863 39.37) (end 46.863 36.957) (width 1) (layer F.Cu) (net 4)))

